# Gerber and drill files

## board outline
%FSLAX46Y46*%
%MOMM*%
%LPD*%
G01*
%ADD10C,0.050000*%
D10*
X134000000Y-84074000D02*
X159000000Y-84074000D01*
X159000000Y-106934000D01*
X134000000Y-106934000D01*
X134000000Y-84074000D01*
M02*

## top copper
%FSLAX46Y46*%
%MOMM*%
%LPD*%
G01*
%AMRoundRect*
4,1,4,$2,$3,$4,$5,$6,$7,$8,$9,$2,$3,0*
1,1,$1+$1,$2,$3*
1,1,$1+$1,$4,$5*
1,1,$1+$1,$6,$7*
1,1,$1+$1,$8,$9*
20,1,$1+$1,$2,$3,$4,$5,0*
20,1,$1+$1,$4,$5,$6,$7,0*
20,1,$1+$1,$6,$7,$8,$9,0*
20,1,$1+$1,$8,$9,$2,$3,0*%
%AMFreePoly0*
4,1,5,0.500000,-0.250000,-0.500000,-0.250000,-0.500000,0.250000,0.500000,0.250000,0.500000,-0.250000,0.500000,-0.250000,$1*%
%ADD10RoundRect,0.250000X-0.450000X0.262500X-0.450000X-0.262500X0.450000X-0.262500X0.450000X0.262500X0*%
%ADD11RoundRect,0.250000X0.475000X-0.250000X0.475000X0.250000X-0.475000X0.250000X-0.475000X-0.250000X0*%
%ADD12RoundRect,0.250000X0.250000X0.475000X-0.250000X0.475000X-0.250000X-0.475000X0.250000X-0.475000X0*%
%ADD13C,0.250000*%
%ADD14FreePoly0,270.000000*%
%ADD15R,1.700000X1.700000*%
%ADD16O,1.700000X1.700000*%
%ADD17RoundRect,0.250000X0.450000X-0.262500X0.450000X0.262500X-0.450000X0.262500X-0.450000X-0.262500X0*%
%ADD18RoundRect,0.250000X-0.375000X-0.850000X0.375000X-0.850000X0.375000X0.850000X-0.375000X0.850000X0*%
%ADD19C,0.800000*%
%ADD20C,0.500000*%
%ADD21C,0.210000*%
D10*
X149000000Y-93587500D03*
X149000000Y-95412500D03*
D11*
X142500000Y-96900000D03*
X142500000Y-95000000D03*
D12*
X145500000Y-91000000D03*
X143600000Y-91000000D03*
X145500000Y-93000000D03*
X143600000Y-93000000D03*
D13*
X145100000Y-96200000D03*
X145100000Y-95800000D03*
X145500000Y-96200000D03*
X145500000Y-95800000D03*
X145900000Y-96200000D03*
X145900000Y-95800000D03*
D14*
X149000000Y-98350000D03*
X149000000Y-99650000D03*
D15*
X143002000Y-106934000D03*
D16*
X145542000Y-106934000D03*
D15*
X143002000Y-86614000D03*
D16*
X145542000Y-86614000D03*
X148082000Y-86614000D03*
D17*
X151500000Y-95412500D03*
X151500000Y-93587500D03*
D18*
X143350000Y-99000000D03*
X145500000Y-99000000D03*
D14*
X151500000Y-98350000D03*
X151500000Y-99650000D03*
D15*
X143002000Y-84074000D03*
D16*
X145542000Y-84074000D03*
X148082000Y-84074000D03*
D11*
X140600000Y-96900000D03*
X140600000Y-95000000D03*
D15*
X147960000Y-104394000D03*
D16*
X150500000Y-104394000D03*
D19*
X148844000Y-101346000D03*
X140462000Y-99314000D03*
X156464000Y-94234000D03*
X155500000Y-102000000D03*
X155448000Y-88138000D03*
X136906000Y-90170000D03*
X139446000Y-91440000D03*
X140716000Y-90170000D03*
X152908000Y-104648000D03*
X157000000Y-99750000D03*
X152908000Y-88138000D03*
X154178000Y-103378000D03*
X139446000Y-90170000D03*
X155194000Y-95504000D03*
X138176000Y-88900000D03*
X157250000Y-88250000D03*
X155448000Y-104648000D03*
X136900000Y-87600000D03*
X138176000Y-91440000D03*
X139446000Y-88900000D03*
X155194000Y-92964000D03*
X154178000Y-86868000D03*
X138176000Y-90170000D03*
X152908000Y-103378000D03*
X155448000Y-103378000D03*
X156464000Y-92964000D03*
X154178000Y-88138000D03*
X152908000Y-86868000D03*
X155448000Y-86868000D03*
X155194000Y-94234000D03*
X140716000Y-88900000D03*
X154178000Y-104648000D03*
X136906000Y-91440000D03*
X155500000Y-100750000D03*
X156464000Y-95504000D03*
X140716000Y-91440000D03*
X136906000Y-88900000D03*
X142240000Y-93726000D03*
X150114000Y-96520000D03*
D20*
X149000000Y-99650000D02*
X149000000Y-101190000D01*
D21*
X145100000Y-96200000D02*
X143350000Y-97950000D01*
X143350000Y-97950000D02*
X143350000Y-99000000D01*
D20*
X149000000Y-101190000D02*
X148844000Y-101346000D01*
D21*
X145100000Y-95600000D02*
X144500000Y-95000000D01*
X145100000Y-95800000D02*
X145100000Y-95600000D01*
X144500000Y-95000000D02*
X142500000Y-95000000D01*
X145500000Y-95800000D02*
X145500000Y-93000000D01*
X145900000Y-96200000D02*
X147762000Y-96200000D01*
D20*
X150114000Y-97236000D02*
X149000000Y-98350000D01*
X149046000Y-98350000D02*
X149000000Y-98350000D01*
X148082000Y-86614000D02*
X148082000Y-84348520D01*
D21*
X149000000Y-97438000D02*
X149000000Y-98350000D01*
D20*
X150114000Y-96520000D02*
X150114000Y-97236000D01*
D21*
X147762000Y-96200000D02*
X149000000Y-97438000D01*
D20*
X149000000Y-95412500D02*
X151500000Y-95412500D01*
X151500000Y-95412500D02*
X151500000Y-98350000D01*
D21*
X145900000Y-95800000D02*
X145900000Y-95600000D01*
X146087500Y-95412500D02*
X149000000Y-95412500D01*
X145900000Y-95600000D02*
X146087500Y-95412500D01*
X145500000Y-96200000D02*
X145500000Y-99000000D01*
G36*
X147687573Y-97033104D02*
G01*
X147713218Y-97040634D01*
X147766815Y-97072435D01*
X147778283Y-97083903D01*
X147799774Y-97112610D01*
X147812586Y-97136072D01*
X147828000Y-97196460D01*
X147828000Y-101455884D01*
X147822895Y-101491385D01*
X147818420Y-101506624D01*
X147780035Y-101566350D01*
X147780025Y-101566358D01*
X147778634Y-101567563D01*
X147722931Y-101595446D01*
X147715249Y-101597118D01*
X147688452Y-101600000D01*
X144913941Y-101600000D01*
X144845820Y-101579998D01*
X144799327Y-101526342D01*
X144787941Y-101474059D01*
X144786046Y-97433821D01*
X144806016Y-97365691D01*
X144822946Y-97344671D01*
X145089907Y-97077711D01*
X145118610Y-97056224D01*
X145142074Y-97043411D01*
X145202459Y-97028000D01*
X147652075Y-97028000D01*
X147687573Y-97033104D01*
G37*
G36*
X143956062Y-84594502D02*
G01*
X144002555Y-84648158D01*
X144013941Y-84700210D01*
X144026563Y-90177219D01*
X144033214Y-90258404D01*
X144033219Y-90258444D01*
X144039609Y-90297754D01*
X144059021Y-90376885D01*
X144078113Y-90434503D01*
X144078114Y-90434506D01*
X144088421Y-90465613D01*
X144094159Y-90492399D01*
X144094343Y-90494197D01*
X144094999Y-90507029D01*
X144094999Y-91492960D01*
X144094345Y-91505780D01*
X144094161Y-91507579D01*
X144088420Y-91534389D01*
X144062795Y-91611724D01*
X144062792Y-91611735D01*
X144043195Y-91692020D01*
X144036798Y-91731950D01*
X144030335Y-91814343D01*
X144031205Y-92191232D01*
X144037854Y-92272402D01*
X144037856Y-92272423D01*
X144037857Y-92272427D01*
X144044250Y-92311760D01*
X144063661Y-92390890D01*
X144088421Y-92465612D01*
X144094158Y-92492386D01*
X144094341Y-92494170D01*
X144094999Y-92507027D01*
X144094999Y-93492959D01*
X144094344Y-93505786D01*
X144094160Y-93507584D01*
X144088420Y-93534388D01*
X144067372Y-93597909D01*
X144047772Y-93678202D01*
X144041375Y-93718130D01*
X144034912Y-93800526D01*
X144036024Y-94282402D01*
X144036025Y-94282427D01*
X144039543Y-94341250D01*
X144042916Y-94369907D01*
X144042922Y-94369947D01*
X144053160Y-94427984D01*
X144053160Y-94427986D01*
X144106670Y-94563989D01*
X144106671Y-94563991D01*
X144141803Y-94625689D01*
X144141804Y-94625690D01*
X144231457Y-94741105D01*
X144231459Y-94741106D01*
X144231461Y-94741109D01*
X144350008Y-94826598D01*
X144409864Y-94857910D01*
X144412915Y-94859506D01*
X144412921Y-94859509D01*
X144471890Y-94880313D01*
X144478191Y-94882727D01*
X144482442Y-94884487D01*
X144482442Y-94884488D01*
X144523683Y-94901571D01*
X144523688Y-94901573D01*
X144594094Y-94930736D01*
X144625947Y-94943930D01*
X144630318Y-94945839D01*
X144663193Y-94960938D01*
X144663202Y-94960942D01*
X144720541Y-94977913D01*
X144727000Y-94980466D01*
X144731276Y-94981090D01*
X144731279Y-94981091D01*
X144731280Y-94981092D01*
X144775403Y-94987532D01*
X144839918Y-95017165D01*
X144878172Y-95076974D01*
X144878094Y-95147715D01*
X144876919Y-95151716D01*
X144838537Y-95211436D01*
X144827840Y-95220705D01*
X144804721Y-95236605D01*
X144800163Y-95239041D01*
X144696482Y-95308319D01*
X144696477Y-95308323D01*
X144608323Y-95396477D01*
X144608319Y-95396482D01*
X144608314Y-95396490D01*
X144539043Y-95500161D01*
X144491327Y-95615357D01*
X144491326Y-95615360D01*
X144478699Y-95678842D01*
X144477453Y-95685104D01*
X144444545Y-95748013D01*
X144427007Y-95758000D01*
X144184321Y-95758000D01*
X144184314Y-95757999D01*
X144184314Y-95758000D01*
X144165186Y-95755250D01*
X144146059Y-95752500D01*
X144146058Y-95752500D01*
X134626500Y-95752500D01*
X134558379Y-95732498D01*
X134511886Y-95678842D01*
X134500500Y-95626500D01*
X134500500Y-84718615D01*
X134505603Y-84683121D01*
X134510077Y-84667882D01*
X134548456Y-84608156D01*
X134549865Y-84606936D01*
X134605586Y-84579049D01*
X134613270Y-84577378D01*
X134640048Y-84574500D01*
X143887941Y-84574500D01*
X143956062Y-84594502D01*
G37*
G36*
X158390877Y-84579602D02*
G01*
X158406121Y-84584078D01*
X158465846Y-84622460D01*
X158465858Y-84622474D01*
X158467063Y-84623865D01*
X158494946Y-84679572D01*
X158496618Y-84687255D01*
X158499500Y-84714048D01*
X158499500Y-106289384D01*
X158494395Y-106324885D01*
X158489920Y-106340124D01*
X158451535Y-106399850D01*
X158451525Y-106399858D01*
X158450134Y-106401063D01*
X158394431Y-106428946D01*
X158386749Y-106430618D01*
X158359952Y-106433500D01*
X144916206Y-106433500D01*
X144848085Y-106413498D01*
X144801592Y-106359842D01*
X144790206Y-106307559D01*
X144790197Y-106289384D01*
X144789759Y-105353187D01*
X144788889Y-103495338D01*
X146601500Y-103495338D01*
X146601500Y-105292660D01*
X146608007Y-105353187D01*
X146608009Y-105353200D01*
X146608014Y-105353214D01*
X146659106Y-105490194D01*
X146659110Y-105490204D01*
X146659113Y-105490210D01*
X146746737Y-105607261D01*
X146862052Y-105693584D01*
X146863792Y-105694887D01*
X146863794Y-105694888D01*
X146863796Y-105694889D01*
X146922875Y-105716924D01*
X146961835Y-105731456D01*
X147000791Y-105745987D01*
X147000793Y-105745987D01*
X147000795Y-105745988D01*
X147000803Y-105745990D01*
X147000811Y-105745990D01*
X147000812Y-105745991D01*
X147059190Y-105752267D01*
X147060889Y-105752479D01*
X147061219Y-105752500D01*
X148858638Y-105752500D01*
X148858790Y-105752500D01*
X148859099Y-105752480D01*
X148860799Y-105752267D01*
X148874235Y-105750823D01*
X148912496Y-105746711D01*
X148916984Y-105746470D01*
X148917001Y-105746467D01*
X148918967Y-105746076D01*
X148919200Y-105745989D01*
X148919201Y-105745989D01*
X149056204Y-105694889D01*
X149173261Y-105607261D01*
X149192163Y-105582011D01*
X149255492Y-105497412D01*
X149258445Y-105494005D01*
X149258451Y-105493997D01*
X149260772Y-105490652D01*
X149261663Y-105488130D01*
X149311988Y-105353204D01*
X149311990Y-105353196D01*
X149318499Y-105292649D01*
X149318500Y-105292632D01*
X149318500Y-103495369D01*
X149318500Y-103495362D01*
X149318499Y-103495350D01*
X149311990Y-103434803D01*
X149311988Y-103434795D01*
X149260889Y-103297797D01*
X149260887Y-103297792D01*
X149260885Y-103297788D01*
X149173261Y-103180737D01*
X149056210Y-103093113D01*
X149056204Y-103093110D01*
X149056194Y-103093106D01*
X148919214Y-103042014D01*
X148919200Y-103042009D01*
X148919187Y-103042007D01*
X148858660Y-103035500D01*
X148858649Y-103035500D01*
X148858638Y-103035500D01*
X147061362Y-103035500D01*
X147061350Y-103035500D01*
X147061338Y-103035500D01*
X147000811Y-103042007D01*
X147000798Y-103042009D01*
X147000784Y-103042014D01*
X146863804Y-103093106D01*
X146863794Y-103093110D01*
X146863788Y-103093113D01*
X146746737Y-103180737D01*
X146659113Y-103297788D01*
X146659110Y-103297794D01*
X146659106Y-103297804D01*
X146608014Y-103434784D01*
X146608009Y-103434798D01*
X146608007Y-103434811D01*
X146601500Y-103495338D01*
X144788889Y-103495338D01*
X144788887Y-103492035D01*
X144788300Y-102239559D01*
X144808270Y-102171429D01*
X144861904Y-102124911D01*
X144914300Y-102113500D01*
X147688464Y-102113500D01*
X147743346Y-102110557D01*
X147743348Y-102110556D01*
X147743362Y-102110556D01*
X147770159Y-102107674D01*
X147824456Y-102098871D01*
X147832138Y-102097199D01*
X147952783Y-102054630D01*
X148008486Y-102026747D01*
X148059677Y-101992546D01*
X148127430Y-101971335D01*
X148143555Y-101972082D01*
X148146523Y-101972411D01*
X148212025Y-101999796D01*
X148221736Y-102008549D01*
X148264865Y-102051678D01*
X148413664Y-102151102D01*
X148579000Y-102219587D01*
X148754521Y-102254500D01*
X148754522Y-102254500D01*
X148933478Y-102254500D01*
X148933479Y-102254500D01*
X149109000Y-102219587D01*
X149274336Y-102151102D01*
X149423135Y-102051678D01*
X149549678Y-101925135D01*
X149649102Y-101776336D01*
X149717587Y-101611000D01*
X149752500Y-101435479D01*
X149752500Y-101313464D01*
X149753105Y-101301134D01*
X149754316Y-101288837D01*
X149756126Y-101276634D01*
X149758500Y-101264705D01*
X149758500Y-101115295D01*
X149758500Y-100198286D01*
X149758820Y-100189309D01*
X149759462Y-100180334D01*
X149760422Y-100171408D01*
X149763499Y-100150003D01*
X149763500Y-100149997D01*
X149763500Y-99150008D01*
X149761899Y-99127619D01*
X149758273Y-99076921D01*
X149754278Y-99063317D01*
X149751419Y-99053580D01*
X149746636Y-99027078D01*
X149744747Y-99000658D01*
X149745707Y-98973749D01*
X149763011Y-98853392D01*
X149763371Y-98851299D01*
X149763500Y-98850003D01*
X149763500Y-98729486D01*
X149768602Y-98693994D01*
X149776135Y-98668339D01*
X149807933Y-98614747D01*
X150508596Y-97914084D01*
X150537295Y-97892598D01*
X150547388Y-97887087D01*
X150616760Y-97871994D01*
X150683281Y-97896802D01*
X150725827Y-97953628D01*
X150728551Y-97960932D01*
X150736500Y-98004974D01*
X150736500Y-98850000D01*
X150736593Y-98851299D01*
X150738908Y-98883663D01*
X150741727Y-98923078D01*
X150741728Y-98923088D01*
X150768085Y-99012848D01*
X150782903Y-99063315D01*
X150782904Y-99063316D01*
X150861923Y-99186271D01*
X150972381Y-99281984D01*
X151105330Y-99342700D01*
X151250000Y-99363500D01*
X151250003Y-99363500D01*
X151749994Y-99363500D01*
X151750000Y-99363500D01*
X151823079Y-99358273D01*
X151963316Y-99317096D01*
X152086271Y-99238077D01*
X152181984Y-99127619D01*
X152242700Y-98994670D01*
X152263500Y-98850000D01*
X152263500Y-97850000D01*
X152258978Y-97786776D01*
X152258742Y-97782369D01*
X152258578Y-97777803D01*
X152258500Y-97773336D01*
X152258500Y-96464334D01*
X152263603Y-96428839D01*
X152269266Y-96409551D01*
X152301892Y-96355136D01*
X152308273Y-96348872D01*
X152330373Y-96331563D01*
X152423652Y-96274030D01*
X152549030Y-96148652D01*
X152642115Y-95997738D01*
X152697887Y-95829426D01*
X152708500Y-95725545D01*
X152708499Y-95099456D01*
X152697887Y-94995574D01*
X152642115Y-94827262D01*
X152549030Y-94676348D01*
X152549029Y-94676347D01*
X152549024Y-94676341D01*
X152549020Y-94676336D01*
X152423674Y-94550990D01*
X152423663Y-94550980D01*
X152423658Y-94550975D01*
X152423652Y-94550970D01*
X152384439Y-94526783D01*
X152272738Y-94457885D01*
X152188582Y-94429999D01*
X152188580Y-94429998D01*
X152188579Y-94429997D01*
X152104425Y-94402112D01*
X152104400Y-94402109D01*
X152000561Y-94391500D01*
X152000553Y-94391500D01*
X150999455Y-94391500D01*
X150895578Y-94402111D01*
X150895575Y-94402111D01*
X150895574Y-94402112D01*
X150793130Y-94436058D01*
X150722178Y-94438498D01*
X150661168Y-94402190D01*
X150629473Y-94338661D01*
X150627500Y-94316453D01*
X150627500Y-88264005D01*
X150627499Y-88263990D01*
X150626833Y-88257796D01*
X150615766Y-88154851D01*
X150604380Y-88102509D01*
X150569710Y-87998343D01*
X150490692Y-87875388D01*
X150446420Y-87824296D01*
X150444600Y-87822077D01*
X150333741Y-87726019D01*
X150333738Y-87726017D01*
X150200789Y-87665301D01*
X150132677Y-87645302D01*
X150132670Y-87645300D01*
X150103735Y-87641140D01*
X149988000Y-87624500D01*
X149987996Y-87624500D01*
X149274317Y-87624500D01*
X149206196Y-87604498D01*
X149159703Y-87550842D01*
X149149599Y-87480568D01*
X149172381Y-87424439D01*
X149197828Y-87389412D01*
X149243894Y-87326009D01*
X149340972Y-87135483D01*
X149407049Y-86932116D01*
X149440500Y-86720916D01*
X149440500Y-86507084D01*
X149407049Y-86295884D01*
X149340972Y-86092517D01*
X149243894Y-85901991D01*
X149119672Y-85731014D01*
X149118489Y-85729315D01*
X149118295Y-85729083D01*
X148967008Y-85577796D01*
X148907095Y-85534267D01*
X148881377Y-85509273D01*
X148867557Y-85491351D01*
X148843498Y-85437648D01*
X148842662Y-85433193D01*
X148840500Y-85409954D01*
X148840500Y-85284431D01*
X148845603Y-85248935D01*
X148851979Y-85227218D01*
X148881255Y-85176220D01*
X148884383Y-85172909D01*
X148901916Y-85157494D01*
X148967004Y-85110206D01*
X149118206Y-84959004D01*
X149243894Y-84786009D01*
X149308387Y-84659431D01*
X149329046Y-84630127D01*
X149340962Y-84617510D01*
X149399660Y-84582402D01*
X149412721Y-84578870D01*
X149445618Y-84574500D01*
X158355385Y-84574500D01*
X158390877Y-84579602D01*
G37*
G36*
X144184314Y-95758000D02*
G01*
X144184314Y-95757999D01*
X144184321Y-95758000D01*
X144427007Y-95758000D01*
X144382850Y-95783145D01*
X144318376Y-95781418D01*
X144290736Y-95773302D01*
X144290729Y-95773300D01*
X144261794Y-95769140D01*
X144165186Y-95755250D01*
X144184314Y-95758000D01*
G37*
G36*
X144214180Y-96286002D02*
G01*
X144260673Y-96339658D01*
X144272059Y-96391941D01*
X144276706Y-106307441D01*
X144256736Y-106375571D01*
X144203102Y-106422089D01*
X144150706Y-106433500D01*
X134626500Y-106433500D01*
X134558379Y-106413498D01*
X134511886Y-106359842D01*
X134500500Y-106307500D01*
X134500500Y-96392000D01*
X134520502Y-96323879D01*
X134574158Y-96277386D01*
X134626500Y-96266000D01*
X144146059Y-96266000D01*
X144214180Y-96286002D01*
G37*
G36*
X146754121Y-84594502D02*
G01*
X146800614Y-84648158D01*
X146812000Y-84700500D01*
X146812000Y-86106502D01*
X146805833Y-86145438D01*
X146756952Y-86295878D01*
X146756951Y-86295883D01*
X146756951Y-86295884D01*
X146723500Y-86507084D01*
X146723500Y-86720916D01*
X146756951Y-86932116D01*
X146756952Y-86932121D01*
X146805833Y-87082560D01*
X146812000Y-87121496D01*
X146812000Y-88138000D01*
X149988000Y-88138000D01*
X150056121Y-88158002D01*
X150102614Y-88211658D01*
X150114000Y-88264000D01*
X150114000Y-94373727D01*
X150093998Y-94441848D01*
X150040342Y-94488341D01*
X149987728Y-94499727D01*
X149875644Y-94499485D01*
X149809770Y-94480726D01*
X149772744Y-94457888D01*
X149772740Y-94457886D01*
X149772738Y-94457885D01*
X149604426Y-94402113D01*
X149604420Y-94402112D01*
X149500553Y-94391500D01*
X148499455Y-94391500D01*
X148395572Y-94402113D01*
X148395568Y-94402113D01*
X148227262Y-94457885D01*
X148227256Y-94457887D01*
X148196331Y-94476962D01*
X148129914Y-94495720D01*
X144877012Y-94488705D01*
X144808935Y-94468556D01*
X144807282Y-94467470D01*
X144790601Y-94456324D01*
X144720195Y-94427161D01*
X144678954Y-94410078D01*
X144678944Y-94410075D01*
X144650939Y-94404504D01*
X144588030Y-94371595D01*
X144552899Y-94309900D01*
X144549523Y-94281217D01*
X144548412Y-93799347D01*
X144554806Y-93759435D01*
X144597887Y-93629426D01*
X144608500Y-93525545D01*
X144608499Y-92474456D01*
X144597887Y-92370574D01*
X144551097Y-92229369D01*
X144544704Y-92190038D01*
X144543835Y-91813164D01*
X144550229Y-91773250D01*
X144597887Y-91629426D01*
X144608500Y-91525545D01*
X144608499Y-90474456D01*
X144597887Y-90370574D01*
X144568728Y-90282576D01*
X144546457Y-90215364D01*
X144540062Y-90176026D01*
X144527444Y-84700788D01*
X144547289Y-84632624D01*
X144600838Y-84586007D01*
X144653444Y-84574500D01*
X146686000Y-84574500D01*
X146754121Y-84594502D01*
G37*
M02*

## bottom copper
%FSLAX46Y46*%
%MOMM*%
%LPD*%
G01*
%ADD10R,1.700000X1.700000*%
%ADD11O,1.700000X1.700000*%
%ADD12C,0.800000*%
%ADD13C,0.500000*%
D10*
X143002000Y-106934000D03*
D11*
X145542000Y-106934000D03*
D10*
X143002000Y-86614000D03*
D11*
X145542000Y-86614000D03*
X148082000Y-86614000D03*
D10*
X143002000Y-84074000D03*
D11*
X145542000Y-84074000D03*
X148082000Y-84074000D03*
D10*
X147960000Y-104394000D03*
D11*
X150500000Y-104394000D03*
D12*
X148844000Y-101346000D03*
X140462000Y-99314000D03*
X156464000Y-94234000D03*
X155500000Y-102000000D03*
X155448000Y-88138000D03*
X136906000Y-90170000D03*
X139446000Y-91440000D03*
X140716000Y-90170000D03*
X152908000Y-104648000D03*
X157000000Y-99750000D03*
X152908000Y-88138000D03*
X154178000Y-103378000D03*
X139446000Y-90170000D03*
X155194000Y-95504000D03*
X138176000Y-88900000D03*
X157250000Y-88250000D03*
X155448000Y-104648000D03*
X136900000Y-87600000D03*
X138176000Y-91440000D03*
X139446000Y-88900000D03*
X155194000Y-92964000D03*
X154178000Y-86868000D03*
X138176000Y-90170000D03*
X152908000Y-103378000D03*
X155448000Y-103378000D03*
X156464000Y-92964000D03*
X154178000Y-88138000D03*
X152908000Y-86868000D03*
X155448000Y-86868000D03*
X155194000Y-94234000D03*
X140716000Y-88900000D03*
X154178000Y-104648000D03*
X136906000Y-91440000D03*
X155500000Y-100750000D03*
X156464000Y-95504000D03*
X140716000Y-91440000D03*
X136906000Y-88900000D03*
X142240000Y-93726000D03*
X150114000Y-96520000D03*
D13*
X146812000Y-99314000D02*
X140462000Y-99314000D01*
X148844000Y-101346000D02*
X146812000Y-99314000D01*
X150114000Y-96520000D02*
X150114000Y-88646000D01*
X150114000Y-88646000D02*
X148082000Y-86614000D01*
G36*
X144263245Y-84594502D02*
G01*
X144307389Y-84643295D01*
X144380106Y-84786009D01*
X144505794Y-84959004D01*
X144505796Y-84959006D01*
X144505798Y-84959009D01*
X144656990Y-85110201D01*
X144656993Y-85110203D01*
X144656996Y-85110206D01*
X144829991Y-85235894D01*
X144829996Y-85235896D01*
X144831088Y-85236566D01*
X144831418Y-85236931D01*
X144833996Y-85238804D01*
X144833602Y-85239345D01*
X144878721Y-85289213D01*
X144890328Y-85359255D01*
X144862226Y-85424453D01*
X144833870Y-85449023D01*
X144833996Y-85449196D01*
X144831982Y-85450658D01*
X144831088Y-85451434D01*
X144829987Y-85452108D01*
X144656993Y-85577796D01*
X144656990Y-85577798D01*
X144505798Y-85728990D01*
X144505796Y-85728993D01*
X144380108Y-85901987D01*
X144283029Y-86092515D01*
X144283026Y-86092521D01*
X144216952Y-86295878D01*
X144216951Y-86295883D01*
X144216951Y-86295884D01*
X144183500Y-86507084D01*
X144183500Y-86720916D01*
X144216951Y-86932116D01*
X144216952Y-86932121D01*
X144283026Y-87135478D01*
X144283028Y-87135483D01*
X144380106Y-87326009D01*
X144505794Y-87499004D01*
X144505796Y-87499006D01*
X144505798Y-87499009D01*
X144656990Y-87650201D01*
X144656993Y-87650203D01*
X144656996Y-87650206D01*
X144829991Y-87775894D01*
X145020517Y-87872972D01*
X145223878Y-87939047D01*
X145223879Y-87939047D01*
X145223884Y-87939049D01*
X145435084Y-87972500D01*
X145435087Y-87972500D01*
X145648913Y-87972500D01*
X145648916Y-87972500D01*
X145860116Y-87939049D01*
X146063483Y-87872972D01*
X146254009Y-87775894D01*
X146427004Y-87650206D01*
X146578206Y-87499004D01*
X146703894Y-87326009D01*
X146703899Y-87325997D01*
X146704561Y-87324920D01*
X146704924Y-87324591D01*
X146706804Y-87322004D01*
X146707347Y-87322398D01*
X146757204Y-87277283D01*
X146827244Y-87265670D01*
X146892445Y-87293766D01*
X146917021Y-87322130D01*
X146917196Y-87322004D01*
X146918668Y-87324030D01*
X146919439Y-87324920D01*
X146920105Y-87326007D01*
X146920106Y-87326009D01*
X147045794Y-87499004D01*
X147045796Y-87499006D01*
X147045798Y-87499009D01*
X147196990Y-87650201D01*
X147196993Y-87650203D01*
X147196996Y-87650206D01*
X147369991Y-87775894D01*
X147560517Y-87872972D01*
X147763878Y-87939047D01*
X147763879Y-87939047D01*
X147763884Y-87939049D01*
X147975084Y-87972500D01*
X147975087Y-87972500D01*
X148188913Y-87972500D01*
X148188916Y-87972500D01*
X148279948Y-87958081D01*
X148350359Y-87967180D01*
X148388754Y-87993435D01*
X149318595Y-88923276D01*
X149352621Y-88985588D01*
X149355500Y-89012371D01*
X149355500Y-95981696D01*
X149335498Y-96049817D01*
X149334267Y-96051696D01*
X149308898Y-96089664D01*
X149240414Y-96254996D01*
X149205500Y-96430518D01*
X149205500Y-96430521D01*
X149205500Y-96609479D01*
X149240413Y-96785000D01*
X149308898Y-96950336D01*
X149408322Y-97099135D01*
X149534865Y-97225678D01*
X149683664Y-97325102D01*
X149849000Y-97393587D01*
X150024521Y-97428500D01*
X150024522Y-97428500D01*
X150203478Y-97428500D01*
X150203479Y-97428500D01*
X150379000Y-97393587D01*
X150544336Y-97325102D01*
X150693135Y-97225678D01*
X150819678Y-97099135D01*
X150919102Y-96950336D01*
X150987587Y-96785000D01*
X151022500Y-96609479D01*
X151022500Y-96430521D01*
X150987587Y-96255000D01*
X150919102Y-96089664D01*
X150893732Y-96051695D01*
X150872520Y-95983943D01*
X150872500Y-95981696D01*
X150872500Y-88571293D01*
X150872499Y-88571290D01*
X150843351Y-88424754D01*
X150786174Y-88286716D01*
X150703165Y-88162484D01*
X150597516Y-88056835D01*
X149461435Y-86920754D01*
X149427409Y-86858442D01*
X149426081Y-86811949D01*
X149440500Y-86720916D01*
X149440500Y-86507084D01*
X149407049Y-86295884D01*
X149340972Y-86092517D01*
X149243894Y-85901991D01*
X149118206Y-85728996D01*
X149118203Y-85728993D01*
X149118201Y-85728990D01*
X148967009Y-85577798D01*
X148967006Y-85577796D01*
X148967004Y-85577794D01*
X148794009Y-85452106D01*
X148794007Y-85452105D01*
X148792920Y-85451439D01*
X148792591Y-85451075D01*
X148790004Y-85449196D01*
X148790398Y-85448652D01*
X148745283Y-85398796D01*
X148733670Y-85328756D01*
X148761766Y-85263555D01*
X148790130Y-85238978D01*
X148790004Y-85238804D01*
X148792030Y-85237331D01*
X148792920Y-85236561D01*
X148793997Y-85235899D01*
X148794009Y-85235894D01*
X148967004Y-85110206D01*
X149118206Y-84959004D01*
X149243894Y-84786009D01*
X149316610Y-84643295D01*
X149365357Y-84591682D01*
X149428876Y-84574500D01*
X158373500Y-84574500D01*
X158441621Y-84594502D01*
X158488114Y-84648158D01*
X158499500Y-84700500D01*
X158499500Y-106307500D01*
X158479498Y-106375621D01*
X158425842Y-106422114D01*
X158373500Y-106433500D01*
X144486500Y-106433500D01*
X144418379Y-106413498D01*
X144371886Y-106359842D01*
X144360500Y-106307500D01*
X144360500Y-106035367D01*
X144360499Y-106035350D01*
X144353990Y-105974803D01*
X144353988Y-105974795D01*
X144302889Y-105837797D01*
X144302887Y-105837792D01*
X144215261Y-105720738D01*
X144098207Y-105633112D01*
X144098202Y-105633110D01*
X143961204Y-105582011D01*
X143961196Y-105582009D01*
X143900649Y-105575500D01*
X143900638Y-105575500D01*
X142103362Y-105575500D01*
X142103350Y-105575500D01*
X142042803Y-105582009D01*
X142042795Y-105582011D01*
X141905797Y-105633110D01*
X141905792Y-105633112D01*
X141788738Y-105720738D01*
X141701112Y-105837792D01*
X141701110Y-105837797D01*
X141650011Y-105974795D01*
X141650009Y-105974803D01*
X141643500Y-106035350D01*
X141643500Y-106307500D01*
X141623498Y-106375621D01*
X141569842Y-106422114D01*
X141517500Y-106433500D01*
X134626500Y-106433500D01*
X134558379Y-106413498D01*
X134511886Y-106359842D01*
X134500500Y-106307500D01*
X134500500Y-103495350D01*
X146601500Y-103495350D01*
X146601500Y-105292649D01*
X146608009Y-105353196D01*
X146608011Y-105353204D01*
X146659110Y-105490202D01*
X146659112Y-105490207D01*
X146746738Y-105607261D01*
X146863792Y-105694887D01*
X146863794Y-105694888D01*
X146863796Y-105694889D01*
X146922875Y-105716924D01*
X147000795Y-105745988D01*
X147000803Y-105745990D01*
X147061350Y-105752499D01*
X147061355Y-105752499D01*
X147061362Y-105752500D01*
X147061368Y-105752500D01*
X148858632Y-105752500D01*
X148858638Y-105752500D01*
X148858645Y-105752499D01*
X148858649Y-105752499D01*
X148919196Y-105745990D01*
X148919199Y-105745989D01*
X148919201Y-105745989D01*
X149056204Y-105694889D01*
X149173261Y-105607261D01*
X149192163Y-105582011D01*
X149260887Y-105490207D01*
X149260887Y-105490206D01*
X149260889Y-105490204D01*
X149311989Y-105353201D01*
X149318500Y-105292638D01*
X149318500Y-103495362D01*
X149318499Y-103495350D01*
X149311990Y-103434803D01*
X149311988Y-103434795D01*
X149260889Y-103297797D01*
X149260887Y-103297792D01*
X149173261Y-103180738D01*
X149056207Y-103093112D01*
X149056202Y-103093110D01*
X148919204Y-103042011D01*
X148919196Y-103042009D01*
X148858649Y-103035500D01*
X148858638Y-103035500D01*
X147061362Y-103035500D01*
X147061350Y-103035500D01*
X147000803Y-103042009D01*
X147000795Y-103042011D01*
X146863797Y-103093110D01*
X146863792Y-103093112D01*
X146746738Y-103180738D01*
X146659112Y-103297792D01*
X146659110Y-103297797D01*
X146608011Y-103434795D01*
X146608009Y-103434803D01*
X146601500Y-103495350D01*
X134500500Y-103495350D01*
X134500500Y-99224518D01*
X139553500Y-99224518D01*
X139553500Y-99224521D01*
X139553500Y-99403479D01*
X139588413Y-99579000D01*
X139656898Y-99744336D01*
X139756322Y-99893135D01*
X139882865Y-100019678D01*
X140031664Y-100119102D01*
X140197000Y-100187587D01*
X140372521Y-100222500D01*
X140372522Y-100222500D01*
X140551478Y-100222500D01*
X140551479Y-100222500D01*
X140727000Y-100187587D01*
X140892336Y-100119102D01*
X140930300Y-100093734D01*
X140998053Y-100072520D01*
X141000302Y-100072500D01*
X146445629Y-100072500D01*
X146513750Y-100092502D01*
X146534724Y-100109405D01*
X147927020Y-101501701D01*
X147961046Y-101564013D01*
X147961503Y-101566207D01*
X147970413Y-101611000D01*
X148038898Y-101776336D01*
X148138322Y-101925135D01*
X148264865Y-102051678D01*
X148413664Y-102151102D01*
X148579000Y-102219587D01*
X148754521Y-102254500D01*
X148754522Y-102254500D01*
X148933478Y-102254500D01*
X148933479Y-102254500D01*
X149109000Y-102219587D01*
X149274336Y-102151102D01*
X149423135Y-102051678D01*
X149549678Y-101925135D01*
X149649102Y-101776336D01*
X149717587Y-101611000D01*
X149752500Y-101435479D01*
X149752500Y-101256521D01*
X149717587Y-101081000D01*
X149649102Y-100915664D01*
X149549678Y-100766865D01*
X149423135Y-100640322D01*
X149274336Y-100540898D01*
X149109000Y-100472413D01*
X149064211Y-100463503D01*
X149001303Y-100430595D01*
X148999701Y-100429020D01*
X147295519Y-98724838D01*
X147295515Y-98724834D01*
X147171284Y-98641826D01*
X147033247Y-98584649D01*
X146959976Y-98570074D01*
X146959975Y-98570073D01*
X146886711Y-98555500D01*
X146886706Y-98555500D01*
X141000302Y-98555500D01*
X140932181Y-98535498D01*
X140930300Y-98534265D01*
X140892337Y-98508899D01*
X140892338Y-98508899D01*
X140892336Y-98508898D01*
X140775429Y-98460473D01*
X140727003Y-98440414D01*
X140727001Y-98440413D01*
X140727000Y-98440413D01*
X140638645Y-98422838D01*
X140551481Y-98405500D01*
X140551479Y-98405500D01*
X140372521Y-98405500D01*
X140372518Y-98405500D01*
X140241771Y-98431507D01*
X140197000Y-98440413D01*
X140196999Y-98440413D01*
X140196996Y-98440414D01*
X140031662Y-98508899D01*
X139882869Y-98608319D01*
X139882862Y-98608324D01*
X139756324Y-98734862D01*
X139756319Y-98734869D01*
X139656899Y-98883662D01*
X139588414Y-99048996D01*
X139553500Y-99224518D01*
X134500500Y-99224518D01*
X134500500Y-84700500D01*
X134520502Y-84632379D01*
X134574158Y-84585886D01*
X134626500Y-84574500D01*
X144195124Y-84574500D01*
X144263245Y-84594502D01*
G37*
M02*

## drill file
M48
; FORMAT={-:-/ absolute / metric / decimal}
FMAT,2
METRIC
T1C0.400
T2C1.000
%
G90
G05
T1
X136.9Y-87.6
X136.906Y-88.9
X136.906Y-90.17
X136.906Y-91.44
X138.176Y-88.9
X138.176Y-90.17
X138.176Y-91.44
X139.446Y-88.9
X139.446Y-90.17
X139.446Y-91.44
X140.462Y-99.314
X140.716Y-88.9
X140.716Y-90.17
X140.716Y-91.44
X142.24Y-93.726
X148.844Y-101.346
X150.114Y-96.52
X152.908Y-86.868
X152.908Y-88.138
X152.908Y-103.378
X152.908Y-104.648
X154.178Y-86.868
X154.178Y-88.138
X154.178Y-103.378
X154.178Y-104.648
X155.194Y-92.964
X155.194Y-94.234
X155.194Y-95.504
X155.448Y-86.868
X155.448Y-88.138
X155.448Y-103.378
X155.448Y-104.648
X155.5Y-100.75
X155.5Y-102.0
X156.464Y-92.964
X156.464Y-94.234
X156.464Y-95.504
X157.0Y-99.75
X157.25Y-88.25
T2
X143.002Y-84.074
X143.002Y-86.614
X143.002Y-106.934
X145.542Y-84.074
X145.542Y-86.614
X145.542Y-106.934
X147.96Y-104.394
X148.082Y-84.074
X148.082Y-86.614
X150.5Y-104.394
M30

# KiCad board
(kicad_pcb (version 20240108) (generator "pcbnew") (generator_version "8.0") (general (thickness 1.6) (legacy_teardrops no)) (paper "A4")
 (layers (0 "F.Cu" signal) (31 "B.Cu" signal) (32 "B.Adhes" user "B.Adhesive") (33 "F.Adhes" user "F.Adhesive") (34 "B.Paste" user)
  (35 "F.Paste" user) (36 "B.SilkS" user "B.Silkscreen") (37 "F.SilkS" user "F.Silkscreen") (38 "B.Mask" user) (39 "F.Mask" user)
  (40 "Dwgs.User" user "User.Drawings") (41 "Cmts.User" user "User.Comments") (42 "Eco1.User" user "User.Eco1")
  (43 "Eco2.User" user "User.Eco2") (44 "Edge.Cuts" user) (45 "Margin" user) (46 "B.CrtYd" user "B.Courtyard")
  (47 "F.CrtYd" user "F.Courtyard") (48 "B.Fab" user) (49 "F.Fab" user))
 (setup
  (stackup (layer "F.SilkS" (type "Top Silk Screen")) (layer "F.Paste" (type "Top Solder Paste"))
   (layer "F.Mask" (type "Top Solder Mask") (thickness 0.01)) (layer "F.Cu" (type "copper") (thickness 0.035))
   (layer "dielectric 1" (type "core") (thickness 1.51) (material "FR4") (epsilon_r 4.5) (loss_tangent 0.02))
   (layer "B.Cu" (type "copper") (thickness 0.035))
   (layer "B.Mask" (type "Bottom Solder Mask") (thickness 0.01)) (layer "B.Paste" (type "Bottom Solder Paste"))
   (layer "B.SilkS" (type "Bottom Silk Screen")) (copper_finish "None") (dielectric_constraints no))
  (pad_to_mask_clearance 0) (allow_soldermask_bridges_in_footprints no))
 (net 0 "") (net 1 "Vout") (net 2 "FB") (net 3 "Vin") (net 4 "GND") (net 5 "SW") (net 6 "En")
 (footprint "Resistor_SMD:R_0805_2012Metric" (layer "F.Cu") (at 149 94.5 -90)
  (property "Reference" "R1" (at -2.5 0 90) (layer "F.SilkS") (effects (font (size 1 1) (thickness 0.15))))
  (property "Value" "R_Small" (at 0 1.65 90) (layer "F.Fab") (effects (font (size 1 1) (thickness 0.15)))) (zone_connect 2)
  (pad "1" smd roundrect (at -0.9125 0 270) (size 1.025 1.4) (layers "F.Cu" "F.Paste" "F.Mask") (roundrect_rratio 0.243902) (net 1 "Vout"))
  (pad "2" smd roundrect (at 0.9125 0 270) (size 1.025 1.4) (layers "F.Cu" "F.Paste" "F.Mask") (roundrect_rratio 0.243902) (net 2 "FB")))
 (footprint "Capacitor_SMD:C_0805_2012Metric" (layer "F.Cu") (at 142.5 95.95 90)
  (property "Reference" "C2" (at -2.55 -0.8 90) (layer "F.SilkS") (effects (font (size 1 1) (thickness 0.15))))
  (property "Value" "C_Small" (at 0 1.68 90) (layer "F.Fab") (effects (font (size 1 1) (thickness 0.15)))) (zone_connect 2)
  (pad "1" smd roundrect (at -0.95 0 90) (size 1 1.45) (layers "F.Cu" "F.Paste" "F.Mask") (roundrect_rratio 0.25) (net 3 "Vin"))
  (pad "2" smd roundrect (at 0.95 0 90) (size 1 1.45) (layers "F.Cu" "F.Paste" "F.Mask") (roundrect_rratio 0.25) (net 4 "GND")))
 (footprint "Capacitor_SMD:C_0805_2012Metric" (layer "F.Cu") (at 144.55 91 180)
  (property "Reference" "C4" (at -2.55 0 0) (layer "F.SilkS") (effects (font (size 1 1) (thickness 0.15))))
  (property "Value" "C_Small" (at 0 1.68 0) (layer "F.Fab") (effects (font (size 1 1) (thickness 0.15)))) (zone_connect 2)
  (pad "1" smd roundrect (at -0.95 0 180) (size 1 1.45) (layers "F.Cu" "F.Paste" "F.Mask") (roundrect_rratio 0.25) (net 1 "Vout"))
  (pad "2" smd roundrect (at 0.95 0 180) (size 1 1.45) (layers "F.Cu" "F.Paste" "F.Mask") (roundrect_rratio 0.25) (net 4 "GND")))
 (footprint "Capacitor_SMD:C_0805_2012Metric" (layer "F.Cu") (at 144.55 93 180)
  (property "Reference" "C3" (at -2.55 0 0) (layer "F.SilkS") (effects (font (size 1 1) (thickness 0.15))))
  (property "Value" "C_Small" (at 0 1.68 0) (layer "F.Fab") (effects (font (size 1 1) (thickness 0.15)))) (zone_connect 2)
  (pad "1" smd roundrect (at -0.95 0 180) (size 1 1.45) (layers "F.Cu" "F.Paste" "F.Mask") (roundrect_rratio 0.25) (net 1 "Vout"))
  (pad "2" smd roundrect (at 0.95 0 180) (size 1 1.45) (layers "F.Cu" "F.Paste" "F.Mask") (roundrect_rratio 0.25) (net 4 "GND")))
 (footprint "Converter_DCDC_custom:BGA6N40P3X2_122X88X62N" (layer "F.Cu") (at 145.5 96 90)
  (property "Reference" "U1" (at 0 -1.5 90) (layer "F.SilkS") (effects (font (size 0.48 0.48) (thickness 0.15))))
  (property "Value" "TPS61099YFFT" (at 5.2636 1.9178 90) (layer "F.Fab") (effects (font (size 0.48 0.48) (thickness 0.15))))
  (pad "A1" smd circle (at -0.2 -0.4 90) (size 0.25 0.25) (layers "F.Cu" "F.Paste" "F.Mask") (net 3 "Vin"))
  (pad "A2" smd circle (at 0.2 -0.4 90) (size 0.25 0.25) (layers "F.Cu" "F.Paste" "F.Mask") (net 4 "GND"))
  (pad "B1" smd circle (at -0.2 0 90) (size 0.25 0.25) (layers "F.Cu" "F.Paste" "F.Mask") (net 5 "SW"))
  (pad "B2" smd circle (at 0.2 0 90) (size 0.25 0.25) (layers "F.Cu" "F.Paste" "F.Mask") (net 1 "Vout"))
  (pad "C1" smd circle (at -0.2 0.4 90) (size 0.25 0.25) (layers "F.Cu" "F.Paste" "F.Mask") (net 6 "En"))
  (pad "C2" smd circle (at 0.2 0.4 90) (size 0.25 0.25) (layers "F.Cu" "F.Paste" "F.Mask") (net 2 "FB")))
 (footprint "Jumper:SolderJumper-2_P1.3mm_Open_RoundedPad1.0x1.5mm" (layer "F.Cu") (at 149 99 -90)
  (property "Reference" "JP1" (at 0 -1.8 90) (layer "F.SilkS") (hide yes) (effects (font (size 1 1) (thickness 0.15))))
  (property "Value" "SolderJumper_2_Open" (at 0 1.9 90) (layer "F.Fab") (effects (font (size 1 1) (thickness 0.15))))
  (pad "1" smd custom (at -0.65 0 270) (size 1 0.5) (layers "F.Cu" "F.Mask") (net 6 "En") (zone_connect 2)
   (options (clearance outline) (anchor rect)) (primitives))
  (pad "2" smd custom (at 0.65 0 270) (size 1 0.5) (layers "F.Cu" "F.Mask") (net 3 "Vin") (zone_connect 2)
   (options (clearance outline) (anchor rect)) (primitives)))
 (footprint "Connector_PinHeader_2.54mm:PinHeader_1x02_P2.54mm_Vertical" (layer "F.Cu") (at 143.002 106.934 90)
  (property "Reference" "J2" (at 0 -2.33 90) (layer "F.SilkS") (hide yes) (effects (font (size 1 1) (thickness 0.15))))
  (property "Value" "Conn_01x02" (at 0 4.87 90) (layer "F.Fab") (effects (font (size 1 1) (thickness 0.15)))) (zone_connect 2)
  (pad "1" thru_hole rect (at 0 0 90) (size 1.7 1.7) (drill 1) (layers "*.Cu" "*.Mask") (remove_unused_layers no) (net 3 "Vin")
   (zone_connect 2))
  (pad "2" thru_hole oval (at 0 2.54 90) (size 1.7 1.7) (drill 1) (layers "*.Cu" "*.Mask") (remove_unused_layers no) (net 4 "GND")
   (zone_connect 2)))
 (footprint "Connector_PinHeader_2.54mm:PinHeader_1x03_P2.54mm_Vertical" (layer "F.Cu") (at 143.002 86.614 90)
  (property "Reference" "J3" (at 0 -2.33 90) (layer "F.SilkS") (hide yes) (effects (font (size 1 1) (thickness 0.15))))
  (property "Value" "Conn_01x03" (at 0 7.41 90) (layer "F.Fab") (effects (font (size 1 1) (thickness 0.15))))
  (pad "1" thru_hole rect (at 0 0 90) (size 1.7 1.7) (drill 1) (layers "*.Cu" "*.Mask") (remove_unused_layers no) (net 4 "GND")
   (zone_connect 2))
  (pad "2" thru_hole oval (at 0 2.54 90) (size 1.7 1.7) (drill 1) (layers "*.Cu" "*.Mask") (remove_unused_layers no) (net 1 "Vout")
   (zone_connect 2))
  (pad "3" thru_hole oval (at 0 5.08 90) (size 1.7 1.7) (drill 1) (layers "*.Cu" "*.Mask") (remove_unused_layers no) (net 6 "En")))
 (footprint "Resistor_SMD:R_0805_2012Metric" (layer "F.Cu") (at 151.5 94.5 90)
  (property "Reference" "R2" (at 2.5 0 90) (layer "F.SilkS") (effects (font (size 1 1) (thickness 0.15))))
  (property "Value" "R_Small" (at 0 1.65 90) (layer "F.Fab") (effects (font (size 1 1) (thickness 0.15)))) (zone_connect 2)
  (pad "1" smd roundrect (at -0.9125 0 90) (size 1.025 1.4) (layers "F.Cu" "F.Paste" "F.Mask") (roundrect_rratio 0.243902) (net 2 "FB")
   (zone_connect 2))
  (pad "2" smd roundrect (at 0.9125 0 90) (size 1.025 1.4) (layers "F.Cu" "F.Paste" "F.Mask") (roundrect_rratio 0.243902) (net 4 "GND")
   (zone_connect 2)))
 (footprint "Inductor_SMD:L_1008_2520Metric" (layer "F.Cu") (at 144.425 99)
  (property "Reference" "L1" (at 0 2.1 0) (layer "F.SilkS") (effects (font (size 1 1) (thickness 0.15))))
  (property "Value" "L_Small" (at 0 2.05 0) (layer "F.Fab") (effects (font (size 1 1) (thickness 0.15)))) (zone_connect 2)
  (pad "1" smd roundrect (at -1.075 0) (size 1.25 2.2) (layers "F.Cu" "F.Paste" "F.Mask") (roundrect_rratio 0.2) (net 3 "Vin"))
  (pad "2" smd roundrect (at 1.075 0) (size 1.25 2.2) (layers "F.Cu" "F.Paste" "F.Mask") (roundrect_rratio 0.2) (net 5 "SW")))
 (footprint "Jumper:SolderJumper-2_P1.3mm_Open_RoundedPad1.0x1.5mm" (layer "F.Cu") (at 151.5 99 -90)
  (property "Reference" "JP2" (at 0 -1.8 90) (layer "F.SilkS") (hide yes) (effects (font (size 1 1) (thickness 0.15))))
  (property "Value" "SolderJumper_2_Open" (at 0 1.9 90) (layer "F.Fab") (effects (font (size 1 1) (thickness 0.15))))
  (pad "1" smd custom (at -0.65 0 270) (size 1 0.5) (layers "F.Cu" "F.Mask") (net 2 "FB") (zone_connect 2)
   (options (clearance outline) (anchor rect)) (primitives))
  (pad "2" smd custom (at 0.65 0 270) (size 1 0.5) (layers "F.Cu" "F.Mask") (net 4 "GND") (zone_connect 2)
   (options (clearance outline) (anchor rect)) (primitives)))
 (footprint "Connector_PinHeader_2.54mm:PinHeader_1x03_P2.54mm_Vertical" (layer "F.Cu") (at 143.002 84.074 90)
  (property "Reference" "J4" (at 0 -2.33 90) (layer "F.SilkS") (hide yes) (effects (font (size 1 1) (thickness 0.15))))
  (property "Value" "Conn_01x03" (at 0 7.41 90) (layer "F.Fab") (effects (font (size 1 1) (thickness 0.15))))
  (pad "1" thru_hole rect (at 0 0 90) (size 1.7 1.7) (drill 1) (layers "*.Cu" "*.Mask") (remove_unused_layers no) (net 4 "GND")
   (zone_connect 2))
  (pad "2" thru_hole oval (at 0 2.54 90) (size 1.7 1.7) (drill 1) (layers "*.Cu" "*.Mask") (remove_unused_layers no) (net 1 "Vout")
   (zone_connect 2))
  (pad "3" thru_hole oval (at 0 5.08 90) (size 1.7 1.7) (drill 1) (layers "*.Cu" "*.Mask") (remove_unused_layers no) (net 6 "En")))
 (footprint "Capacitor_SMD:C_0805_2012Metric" (layer "F.Cu") (at 140.6 95.95 90)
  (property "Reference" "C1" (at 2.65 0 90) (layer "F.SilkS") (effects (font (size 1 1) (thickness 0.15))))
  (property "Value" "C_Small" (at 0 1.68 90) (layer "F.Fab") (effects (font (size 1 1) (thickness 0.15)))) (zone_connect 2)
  (pad "1" smd roundrect (at -0.95 0 90) (size 1 1.45) (layers "F.Cu" "F.Paste" "F.Mask") (roundrect_rratio 0.25) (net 3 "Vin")
   (zone_connect 2))
  (pad "2" smd roundrect (at 0.95 0 90) (size 1 1.45) (layers "F.Cu" "F.Paste" "F.Mask") (roundrect_rratio 0.25) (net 4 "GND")
   (zone_connect 2)))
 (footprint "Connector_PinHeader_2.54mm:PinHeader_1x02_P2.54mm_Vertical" (layer "F.Cu") (at 147.96 104.394 90)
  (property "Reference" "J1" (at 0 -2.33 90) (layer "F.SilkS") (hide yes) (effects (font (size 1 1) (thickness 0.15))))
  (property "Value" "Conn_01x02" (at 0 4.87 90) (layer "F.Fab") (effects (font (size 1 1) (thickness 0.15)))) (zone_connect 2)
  (pad "1" thru_hole rect (at 0 0 90) (size 1.7 1.7) (drill 1) (layers "*.Cu" "*.Mask") (remove_unused_layers no) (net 3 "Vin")
   (zone_connect 2))
  (pad "2" thru_hole oval (at 0 2.54 90) (size 1.7 1.7) (drill 1) (layers "*.Cu" "*.Mask") (remove_unused_layers no) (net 4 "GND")
   (zone_connect 2)))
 (gr_rect (start 134 84.074) (end 159 106.934) (stroke (width 0.05) (type solid)) (fill none) (layer "Edge.Cuts"))
 (segment (start 149 99.65) (end 149 101.19) (width 0.5) (layer "F.Cu") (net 3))
 (segment (start 145.1 96.2) (end 143.35 97.95) (width 0.21) (layer "F.Cu") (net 3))
 (segment (start 143.35 97.95) (end 143.35 99) (width 0.21) (layer "F.Cu") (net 3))
 (segment (start 149 101.19) (end 148.844 101.346) (width 0.5) (layer "F.Cu") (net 3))
 (via (at 148.844 101.346) (size 0.8) (drill 0.4) (layers "F.Cu" "B.Cu") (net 3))
 (via (at 140.462 99.314) (size 0.8) (drill 0.4) (layers "F.Cu" "B.Cu") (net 3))
 (segment (start 146.812 99.314) (end 140.462 99.314) (width 0.5) (layer "B.Cu") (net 3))
 (segment (start 148.844 101.346) (end 146.812 99.314) (width 0.5) (layer "B.Cu") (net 3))
 (segment (start 145.1 95.6) (end 144.5 95) (width 0.21) (layer "F.Cu") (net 4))
 (segment (start 145.1 95.8) (end 145.1 95.6) (width 0.21) (layer "F.Cu") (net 4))
 (segment (start 144.5 95) (end 142.5 95) (width 0.21) (layer "F.Cu") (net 4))
 (via (at 156.464 94.234) (size 0.8) (drill 0.4) (layers "F.Cu" "B.Cu") (free yes) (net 4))
 (via (at 155.5 102) (size 0.8) (drill 0.4) (layers "F.Cu" "B.Cu") (free yes) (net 4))
 (via (at 155.448 88.138) (size 0.8) (drill 0.4) (layers "F.Cu" "B.Cu") (free yes) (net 4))
 (via (at 136.906 90.17) (size 0.8) (drill 0.4) (layers "F.Cu" "B.Cu") (free yes) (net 4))
 (via (at 139.446 91.44) (size 0.8) (drill 0.4) (layers "F.Cu" "B.Cu") (free yes) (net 4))
 (via (at 140.716 90.17) (size 0.8) (drill 0.4) (layers "F.Cu" "B.Cu") (free yes) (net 4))
 (via (at 152.908 104.648) (size 0.8) (drill 0.4) (layers "F.Cu" "B.Cu") (free yes) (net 4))
 (via (at 157 99.75) (size 0.8) (drill 0.4) (layers "F.Cu" "B.Cu") (free yes) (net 4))
 (via (at 152.908 88.138) (size 0.8) (drill 0.4) (layers "F.Cu" "B.Cu") (free yes) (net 4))
 (via (at 154.178 103.378) (size 0.8) (drill 0.4) (layers "F.Cu" "B.Cu") (free yes) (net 4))
 (via (at 139.446 90.17) (size 0.8) (drill 0.4) (layers "F.Cu" "B.Cu") (free yes) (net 4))
 (via (at 155.194 95.504) (size 0.8) (drill 0.4) (layers "F.Cu" "B.Cu") (free yes) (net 4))
 (via (at 138.176 88.9) (size 0.8) (drill 0.4) (layers "F.Cu" "B.Cu") (free yes) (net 4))
 (via (at 157.25 88.25) (size 0.8) (drill 0.4) (layers "F.Cu" "B.Cu") (free yes) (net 4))
 (via (at 155.448 104.648) (size 0.8) (drill 0.4) (layers "F.Cu" "B.Cu") (free yes) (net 4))
 (via (at 136.9 87.6) (size 0.8) (drill 0.4) (layers "F.Cu" "B.Cu") (free yes) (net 4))
 (via (at 138.176 91.44) (size 0.8) (drill 0.4) (layers "F.Cu" "B.Cu") (free yes) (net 4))
 (via (at 139.446 88.9) (size 0.8) (drill 0.4) (layers "F.Cu" "B.Cu") (free yes) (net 4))
 (via (at 155.194 92.964) (size 0.8) (drill 0.4) (layers "F.Cu" "B.Cu") (free yes) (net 4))
 (via (at 154.178 86.868) (size 0.8) (drill 0.4) (layers "F.Cu" "B.Cu") (free yes) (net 4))
 (via (at 138.176 90.17) (size 0.8) (drill 0.4) (layers "F.Cu" "B.Cu") (free yes) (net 4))
 (via (at 152.908 103.378) (size 0.8) (drill 0.4) (layers "F.Cu" "B.Cu") (free yes) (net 4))
 (via (at 155.448 103.378) (size 0.8) (drill 0.4) (layers "F.Cu" "B.Cu") (free yes) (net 4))
 (via (at 156.464 92.964) (size 0.8) (drill 0.4) (layers "F.Cu" "B.Cu") (free yes) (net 4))
 (via (at 154.178 88.138) (size 0.8) (drill 0.4) (layers "F.Cu" "B.Cu") (free yes) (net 4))
 (via (at 152.908 86.868) (size 0.8) (drill 0.4) (layers "F.Cu" "B.Cu") (free yes) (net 4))
 (via (at 155.448 86.868) (size 0.8) (drill 0.4) (layers "F.Cu" "B.Cu") (free yes) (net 4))
 (via (at 155.194 94.234) (size 0.8) (drill 0.4) (layers "F.Cu" "B.Cu") (free yes) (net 4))
 (via (at 140.716 88.9) (size 0.8) (drill 0.4) (layers "F.Cu" "B.Cu") (free yes) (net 4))
 (via (at 154.178 104.648) (size 0.8) (drill 0.4) (layers "F.Cu" "B.Cu") (free yes) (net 4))
 (via (at 136.906 91.44) (size 0.8) (drill 0.4) (layers "F.Cu" "B.Cu") (free yes) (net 4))
 (via (at 155.5 100.75) (size 0.8) (drill 0.4) (layers "F.Cu" "B.Cu") (free yes) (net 4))
 (via (at 156.464 95.504) (size 0.8) (drill 0.4) (layers "F.Cu" "B.Cu") (free yes) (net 4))
 (via (at 140.716 91.44) (size 0.8) (drill 0.4) (layers "F.Cu" "B.Cu") (free yes) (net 4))
 (via (at 136.906 88.9) (size 0.8) (drill 0.4) (layers "F.Cu" "B.Cu") (free yes) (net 4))
 (via (at 142.24 93.726) (size 0.8) (drill 0.4) (layers "F.Cu" "B.Cu") (free yes) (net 4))
 (segment (start 145.5 95.8) (end 145.5 93) (width 0.21) (layer "F.Cu") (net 1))
 (segment (start 145.9 96.2) (end 147.762 96.2) (width 0.21) (layer "F.Cu") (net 6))
 (segment (start 150.114 97.236) (end 149 98.35) (width 0.5) (layer "F.Cu") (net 6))
 (segment (start 149.046 98.35) (end 149 98.35) (width 0.5) (layer "F.Cu") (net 6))
 (segment (start 148.082 86.614) (end 148.082 84.34852) (width 0.5) (layer "F.Cu") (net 6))
 (segment (start 149 97.438) (end 149 98.35) (width 0.21) (layer "F.Cu") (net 6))
 (segment (start 150.114 96.52) (end 150.114 97.236) (width 0.5) (layer "F.Cu") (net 6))
 (segment (start 147.762 96.2) (end 149 97.438) (width 0.21) (layer "F.Cu") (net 6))
 (via (at 150.114 96.52) (size 0.8) (drill 0.4) (layers "F.Cu" "B.Cu") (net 6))
 (segment (start 150.114 96.52) (end 150.114 88.646) (width 0.5) (layer "B.Cu") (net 6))
 (segment (start 150.114 88.646) (end 148.082 86.614) (width 0.5) (layer "B.Cu") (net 6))
 (segment (start 149 95.4125) (end 151.5 95.4125) (width 0.5) (layer "F.Cu") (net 2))
 (segment (start 151.5 95.4125) (end 151.5 98.35) (width 0.5) (layer "F.Cu") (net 2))
 (segment (start 145.9 95.8) (end 145.9 95.6) (width 0.21) (layer "F.Cu") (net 2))
 (segment (start 146.0875 95.4125) (end 149 95.4125) (width 0.21) (layer "F.Cu") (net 2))
 (segment (start 145.9 95.6) (end 146.0875 95.4125) (width 0.21) (layer "F.Cu") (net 2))
 (segment (start 145.5 96.2) (end 145.5 99) (width 0.21) (layer "F.Cu") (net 5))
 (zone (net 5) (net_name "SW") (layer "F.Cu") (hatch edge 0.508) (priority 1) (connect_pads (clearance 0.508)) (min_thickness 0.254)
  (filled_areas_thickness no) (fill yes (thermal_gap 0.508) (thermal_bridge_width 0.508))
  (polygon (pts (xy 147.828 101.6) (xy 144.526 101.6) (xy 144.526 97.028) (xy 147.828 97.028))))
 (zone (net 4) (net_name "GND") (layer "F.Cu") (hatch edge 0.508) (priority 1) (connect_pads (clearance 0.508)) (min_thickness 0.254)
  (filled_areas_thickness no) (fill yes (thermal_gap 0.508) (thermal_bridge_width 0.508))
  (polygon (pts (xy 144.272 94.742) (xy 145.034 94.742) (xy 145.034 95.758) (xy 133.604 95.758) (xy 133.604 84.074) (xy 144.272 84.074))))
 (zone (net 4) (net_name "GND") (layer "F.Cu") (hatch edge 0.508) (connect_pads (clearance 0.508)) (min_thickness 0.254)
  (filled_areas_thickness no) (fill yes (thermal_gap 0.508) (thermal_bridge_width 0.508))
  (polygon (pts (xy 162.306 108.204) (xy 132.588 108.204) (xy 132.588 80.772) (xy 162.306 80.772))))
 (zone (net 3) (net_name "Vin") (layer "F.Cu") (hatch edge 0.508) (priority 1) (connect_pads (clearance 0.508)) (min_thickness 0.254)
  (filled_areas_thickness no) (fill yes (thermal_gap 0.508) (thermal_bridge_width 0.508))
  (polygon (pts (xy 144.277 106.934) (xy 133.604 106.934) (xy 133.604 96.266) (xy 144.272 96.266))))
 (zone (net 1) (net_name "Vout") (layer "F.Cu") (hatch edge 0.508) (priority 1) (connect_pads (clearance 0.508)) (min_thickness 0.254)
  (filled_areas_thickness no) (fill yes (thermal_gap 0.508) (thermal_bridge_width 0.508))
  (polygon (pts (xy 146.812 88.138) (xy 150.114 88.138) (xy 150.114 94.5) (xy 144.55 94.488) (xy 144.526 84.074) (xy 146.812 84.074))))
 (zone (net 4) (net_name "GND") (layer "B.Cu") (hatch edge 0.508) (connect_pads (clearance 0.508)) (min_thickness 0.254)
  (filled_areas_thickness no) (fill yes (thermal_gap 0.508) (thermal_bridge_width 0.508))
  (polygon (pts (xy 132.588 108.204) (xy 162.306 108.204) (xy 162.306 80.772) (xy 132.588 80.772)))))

